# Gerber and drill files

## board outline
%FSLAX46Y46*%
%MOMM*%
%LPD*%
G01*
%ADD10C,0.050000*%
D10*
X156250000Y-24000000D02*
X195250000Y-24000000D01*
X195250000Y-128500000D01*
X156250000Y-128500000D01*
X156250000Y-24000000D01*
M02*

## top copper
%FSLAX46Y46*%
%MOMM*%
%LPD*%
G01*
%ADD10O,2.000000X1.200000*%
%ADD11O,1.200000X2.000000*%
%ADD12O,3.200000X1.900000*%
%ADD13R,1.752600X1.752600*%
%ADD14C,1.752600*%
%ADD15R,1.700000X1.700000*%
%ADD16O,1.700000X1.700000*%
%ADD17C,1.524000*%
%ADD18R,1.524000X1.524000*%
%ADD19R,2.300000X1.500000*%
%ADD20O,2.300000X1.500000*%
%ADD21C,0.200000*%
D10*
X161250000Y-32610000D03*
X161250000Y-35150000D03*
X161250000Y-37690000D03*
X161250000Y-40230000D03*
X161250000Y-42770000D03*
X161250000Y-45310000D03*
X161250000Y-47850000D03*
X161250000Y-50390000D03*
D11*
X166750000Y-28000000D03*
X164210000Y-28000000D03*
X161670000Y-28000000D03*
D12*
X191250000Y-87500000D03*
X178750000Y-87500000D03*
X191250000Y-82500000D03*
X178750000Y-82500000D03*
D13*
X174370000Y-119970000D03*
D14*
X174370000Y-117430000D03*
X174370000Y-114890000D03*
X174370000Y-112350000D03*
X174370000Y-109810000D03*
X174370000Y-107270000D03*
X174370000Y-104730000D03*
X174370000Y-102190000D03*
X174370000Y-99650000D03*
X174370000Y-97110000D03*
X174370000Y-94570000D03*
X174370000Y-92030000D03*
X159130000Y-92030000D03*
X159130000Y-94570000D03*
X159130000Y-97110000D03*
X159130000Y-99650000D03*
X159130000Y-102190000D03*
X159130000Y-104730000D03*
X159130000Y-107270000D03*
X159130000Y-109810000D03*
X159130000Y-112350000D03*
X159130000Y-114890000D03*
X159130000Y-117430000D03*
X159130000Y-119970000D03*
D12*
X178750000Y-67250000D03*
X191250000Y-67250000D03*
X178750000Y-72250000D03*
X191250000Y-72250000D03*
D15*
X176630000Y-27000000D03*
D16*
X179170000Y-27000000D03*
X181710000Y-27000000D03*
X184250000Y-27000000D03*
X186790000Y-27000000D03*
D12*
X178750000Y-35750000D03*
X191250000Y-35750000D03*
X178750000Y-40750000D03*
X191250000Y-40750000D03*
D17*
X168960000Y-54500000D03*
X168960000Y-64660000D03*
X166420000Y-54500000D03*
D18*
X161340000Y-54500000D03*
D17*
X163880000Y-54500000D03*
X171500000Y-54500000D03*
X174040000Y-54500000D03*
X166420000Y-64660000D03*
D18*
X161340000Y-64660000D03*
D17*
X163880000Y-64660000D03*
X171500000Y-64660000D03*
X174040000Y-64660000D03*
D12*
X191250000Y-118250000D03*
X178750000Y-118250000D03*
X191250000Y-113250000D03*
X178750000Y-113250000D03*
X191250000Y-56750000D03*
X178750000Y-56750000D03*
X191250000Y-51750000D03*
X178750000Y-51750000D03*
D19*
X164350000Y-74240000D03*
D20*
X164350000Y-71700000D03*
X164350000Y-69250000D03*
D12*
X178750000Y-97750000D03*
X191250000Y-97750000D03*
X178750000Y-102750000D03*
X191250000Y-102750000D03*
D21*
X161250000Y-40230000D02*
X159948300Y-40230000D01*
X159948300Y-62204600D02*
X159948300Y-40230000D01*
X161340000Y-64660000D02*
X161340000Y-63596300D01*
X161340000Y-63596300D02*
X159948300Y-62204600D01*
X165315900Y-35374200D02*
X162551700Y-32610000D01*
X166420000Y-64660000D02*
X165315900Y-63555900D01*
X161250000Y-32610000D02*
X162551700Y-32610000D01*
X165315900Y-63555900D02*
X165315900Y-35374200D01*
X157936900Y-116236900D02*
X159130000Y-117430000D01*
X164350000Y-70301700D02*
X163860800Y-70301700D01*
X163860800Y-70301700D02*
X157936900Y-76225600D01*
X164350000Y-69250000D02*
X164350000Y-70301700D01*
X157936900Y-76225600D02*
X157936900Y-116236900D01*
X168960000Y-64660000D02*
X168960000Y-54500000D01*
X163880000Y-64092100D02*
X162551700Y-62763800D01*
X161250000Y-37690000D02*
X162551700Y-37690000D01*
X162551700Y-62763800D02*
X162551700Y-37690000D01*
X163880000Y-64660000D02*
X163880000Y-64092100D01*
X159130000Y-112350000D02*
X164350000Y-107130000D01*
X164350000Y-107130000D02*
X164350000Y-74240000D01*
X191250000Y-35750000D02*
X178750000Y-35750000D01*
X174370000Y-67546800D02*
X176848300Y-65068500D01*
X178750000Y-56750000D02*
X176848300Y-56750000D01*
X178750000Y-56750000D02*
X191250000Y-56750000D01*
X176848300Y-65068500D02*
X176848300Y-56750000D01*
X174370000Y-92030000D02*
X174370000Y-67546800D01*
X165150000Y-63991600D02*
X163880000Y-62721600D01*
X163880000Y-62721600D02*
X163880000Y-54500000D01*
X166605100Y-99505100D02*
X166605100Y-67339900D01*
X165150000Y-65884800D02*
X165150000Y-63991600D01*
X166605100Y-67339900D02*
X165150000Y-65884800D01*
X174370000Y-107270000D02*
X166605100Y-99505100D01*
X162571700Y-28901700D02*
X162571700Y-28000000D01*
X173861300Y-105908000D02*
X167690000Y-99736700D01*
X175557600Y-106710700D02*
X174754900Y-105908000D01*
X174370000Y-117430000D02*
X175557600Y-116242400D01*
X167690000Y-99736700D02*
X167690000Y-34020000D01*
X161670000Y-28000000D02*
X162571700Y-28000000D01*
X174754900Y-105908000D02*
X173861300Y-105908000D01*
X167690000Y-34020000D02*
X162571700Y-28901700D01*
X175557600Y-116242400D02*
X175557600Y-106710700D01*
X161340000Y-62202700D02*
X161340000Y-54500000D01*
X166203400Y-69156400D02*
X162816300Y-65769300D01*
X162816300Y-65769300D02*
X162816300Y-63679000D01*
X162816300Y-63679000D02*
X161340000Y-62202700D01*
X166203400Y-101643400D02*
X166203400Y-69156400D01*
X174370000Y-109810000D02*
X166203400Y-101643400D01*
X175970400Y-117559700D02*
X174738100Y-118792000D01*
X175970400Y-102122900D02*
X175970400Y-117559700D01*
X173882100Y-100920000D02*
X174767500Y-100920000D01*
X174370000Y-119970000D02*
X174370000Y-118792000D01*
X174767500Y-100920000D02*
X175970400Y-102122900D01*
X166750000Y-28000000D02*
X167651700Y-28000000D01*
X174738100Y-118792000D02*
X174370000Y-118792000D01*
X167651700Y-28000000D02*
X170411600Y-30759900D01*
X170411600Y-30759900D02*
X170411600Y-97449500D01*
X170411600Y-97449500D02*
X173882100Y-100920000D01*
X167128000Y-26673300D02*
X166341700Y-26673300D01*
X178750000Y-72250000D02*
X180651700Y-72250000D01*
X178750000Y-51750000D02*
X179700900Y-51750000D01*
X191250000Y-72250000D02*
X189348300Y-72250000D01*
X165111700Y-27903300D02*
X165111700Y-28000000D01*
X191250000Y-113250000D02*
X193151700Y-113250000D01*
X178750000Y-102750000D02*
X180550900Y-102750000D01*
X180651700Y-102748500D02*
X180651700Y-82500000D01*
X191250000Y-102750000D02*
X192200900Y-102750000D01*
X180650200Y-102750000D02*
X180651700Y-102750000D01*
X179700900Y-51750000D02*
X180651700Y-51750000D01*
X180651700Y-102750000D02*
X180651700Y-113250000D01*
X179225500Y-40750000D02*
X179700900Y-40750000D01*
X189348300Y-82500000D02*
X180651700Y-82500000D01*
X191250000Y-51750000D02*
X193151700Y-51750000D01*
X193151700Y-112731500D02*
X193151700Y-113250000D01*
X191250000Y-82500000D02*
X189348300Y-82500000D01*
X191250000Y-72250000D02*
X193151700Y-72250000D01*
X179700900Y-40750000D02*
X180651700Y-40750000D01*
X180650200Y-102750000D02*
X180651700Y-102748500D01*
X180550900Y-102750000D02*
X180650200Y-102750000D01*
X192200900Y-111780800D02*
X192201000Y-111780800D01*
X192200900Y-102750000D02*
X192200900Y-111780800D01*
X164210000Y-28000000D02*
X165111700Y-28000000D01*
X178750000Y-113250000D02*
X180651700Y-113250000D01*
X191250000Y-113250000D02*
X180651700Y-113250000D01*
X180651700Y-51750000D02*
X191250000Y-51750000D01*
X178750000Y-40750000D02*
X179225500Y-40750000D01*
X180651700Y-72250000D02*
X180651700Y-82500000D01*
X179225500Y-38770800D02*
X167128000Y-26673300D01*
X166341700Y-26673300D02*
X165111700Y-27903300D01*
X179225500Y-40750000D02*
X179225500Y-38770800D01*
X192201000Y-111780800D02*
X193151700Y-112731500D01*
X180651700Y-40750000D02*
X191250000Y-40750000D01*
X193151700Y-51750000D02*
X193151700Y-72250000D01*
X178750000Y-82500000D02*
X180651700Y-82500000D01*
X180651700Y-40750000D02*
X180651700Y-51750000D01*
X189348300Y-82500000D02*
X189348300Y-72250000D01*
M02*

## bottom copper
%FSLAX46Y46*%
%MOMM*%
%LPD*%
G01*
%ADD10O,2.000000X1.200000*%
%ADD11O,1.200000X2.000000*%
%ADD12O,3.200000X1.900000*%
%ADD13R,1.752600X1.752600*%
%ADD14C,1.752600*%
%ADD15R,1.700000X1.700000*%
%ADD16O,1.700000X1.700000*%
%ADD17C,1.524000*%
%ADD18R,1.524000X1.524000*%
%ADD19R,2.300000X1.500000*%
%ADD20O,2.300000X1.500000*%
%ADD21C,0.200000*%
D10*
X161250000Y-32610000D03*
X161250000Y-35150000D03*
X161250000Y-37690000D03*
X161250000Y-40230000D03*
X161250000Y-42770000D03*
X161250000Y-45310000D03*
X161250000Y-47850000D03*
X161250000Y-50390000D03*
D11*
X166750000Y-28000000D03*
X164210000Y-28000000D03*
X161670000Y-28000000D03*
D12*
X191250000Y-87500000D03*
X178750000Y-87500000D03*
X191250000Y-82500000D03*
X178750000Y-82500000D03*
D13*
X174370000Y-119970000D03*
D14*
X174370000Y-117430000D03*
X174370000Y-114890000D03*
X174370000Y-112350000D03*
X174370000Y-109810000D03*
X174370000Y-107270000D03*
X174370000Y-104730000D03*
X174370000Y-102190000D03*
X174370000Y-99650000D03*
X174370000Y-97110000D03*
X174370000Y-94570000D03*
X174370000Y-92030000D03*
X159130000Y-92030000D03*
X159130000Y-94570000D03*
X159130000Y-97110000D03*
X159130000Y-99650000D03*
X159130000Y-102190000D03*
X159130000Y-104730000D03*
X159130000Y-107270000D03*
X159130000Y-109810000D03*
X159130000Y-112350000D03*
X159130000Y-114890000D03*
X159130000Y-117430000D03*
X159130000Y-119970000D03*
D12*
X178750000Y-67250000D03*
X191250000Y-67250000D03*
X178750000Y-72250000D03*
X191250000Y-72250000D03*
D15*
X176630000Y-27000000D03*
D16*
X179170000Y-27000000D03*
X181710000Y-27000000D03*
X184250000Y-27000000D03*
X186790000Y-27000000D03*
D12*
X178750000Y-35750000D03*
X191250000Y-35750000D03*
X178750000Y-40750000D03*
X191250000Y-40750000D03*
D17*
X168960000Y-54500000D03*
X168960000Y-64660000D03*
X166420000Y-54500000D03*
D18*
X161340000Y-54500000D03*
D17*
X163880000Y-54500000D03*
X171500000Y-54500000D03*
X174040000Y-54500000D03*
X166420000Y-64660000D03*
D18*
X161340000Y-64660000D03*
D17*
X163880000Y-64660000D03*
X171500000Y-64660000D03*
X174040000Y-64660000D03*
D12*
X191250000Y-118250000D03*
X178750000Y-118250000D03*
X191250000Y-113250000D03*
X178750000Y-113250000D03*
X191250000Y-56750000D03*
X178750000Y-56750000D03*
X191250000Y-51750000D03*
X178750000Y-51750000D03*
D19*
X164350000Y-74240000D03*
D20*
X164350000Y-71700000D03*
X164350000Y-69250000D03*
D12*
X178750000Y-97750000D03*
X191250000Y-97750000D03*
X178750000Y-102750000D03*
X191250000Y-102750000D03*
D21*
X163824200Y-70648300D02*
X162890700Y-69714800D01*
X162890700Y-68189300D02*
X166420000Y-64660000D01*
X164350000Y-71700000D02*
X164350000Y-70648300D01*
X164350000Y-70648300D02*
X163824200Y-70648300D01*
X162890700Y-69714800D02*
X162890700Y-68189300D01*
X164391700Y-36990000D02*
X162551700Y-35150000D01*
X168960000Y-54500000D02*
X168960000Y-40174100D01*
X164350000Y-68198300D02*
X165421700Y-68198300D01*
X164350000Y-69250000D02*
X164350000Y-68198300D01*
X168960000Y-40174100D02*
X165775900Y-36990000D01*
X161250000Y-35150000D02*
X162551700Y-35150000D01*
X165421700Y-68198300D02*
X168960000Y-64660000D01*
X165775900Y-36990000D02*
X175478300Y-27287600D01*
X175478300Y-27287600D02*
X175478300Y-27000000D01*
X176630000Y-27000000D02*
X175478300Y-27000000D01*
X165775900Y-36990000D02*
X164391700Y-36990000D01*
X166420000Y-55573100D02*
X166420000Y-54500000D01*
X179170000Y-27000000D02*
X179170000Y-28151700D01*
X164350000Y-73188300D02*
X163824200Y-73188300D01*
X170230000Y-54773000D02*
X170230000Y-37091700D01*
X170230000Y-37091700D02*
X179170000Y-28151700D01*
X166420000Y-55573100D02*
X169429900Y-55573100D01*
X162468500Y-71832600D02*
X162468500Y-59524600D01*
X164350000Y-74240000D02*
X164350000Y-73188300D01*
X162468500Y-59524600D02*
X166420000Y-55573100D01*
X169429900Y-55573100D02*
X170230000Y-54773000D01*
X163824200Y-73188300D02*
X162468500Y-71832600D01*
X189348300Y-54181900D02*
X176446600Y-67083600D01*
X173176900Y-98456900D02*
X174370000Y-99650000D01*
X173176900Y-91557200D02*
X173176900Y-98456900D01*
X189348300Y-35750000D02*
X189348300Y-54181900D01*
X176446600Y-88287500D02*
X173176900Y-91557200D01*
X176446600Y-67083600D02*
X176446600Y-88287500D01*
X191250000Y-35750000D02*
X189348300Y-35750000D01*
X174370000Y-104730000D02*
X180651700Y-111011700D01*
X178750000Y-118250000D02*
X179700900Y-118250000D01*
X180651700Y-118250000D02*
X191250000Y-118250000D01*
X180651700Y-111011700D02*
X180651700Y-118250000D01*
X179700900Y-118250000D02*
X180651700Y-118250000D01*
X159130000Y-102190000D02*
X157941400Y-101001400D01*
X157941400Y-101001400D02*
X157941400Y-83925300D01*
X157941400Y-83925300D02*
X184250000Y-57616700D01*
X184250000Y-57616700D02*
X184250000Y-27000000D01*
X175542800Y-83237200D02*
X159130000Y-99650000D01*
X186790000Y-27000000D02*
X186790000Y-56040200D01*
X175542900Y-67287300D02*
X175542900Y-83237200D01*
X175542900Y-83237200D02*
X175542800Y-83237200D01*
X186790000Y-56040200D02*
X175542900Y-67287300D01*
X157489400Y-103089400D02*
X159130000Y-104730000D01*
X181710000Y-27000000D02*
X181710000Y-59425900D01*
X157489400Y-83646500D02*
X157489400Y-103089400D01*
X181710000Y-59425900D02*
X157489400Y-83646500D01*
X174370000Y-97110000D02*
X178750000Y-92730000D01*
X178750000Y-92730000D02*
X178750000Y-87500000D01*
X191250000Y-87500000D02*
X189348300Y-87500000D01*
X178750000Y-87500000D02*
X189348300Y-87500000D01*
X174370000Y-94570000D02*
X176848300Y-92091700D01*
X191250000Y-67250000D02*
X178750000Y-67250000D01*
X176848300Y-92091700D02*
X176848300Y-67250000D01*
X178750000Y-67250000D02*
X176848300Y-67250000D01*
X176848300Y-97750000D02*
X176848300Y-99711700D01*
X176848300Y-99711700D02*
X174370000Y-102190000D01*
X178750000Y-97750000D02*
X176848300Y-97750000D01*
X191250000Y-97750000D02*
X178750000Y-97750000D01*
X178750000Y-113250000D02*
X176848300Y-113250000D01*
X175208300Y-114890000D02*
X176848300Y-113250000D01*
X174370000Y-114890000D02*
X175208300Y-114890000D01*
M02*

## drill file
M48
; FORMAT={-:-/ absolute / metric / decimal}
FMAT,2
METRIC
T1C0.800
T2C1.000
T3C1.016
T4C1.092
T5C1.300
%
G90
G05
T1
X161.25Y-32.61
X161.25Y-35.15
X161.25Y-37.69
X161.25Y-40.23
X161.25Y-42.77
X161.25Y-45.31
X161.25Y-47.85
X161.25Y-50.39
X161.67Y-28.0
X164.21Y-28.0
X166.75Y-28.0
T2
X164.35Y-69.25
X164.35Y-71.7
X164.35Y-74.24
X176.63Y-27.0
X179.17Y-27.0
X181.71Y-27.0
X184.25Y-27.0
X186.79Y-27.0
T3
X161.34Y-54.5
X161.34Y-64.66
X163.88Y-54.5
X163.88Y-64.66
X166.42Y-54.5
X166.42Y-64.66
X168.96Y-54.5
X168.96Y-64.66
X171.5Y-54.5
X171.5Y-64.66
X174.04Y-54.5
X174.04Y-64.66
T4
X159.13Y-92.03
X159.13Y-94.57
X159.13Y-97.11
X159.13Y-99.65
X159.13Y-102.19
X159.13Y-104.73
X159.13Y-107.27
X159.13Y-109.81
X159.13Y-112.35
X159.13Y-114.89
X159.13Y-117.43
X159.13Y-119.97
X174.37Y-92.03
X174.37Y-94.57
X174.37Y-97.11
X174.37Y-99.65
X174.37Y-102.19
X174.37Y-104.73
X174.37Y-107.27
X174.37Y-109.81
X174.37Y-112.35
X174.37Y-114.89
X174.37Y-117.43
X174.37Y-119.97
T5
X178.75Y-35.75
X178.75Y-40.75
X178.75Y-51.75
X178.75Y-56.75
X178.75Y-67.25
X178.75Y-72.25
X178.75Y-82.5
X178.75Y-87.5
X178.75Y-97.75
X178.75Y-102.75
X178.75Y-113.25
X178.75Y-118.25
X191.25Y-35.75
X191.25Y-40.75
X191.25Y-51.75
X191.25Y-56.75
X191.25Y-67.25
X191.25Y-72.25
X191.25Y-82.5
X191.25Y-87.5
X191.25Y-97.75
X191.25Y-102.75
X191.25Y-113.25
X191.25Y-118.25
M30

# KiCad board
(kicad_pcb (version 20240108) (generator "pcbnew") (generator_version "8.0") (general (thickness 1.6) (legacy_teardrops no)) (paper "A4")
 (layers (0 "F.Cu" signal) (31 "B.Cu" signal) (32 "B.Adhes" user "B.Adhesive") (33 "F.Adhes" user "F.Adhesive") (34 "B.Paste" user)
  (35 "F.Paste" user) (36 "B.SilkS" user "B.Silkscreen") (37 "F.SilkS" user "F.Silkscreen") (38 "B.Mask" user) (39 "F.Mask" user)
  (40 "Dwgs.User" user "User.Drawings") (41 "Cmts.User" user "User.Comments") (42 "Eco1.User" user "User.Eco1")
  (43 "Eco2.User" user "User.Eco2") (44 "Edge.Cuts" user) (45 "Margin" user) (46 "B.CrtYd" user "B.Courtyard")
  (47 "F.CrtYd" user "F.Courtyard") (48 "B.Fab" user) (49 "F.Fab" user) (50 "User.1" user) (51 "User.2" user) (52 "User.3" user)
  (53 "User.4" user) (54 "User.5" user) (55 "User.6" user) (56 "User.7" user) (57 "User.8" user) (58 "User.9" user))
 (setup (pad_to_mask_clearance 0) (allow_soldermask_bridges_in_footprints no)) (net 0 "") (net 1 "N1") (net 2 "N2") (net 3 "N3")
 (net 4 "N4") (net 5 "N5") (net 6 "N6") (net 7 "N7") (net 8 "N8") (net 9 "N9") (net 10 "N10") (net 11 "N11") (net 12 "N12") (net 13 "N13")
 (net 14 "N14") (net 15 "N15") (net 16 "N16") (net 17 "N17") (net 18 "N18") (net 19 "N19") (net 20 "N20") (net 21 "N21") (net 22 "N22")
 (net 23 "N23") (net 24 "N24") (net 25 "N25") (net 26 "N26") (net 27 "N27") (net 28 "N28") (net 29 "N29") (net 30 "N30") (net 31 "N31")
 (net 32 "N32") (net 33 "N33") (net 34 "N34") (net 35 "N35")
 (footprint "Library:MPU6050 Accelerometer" (layer "F.Cu") (at 167.75 43.75)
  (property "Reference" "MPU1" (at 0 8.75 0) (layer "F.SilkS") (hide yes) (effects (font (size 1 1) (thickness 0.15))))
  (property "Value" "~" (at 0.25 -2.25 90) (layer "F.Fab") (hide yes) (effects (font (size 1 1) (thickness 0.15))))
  (pad "1" thru_hole oval (at -6.5 -11.14 270) (size 1.2 2) (drill 0.8) (layers "*.Cu" "*.Mask") (remove_unused_layers no) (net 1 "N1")
   (thermal_bridge_angle 45))
  (pad "2" thru_hole oval (at -6.5 -8.6 270) (size 1.2 2) (drill 0.8) (layers "*.Cu" "*.Mask") (remove_unused_layers no) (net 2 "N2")
   (thermal_bridge_angle 45))
  (pad "3" thru_hole oval (at -6.5 -6.06 270) (size 1.2 2) (drill 0.8) (layers "*.Cu" "*.Mask") (remove_unused_layers no) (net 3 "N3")
   (thermal_bridge_angle 45))
  (pad "4" thru_hole oval (at -6.5 -3.52 270) (size 1.2 2) (drill 0.8) (layers "*.Cu" "*.Mask") (remove_unused_layers no) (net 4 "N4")
   (thermal_bridge_angle 45))
  (pad "5" thru_hole oval (at -6.5 -0.98 270) (size 1.2 2) (drill 0.8) (layers "*.Cu" "*.Mask") (remove_unused_layers no) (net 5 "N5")
   (thermal_bridge_angle 45))
  (pad "6" thru_hole oval (at -6.5 1.56 270) (size 1.2 2) (drill 0.8) (layers "*.Cu" "*.Mask") (remove_unused_layers no) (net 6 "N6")
   (thermal_bridge_angle 45))
  (pad "7" thru_hole oval (at -6.5 4.1 270) (size 1.2 2) (drill 0.8) (layers "*.Cu" "*.Mask") (remove_unused_layers no) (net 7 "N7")
   (thermal_bridge_angle 45))
  (pad "8" thru_hole oval (at -6.5 6.64 270) (size 1.2 2) (drill 0.8) (layers "*.Cu" "*.Mask") (remove_unused_layers no) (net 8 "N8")
   (thermal_bridge_angle 45)))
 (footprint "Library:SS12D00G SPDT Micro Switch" (layer "F.Cu") (at 164.21 28 180)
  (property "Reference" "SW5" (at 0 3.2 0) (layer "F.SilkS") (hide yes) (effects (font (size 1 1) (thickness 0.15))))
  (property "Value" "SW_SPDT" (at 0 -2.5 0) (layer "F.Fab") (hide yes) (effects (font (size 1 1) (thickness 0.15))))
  (pad "1" thru_hole oval (at -2.54 0 180) (size 1.2 2) (drill 0.8) (layers "*.Cu" "*.Mask") (remove_unused_layers no) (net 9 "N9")
   (thermal_bridge_angle 45))
  (pad "2" thru_hole oval (at 0 0 180) (size 1.2 2) (drill 0.8) (layers "*.Cu" "*.Mask") (remove_unused_layers no) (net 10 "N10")
   (thermal_bridge_angle 45))
  (pad "3" thru_hole oval (at 2.54 0 180) (size 1.2 2) (drill 0.8) (layers "*.Cu" "*.Mask") (remove_unused_layers no) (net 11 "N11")
   (thermal_bridge_angle 45)))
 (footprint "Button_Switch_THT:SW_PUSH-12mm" (layer "F.Cu") (at 191.25 87.5 180)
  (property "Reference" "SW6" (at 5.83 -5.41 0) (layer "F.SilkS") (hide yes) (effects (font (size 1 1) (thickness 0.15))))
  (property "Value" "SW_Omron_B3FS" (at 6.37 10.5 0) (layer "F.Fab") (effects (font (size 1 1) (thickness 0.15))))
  (pad "1" thru_hole oval (at 0 0 180) (size 3.2 1.9) (drill 1.3) (layers "*.Cu" "*.Mask") (remove_unused_layers no) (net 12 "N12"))
  (pad "1" thru_hole oval (at 12.5 0 180) (size 3.2 1.9) (drill 1.3) (layers "*.Cu" "*.Mask") (remove_unused_layers no) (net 12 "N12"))
  (pad "2" thru_hole oval (at 0 5 180) (size 3.2 1.9) (drill 1.3) (layers "*.Cu" "*.Mask") (remove_unused_layers no) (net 10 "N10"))
  (pad "2" thru_hole oval (at 12.5 5 180) (size 3.2 1.9) (drill 1.3) (layers "*.Cu" "*.Mask") (remove_unused_layers no) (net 10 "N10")))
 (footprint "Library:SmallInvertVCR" (layer "F.Cu") (at 167 83.5)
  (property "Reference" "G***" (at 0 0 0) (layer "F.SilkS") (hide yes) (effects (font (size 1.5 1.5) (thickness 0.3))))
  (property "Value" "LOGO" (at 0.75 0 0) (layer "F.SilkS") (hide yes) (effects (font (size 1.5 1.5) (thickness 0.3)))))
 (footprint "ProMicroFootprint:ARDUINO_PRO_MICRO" (layer "F.Cu") (at 166.75 106 90)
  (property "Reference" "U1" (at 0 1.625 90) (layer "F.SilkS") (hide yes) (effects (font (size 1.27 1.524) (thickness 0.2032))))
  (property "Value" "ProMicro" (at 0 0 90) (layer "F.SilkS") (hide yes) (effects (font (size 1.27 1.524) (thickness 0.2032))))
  (pad "1" thru_hole rect (at -13.97 7.62 90) (size 1.7526 1.7526) (drill 1.0922) (layers "*.Cu" "*.SilkS" "*.Mask")
   (remove_unused_layers no) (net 9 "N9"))
  (pad "2" thru_hole circle (at -11.43 7.62 90) (size 1.7526 1.7526) (drill 1.0922) (layers "*.Cu" "*.SilkS" "*.Mask")
   (remove_unused_layers no) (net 11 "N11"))
  (pad "3" thru_hole circle (at -8.89 7.62 90) (size 1.7526 1.7526) (drill 1.0922) (layers "*.Cu" "*.SilkS" "*.Mask")
   (remove_unused_layers no) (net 10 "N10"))
  (pad "4" thru_hole circle (at -6.35 7.62 90) (size 1.7526 1.7526) (drill 1.0922) (layers "*.Cu" "*.SilkS" "*.Mask")
   (remove_unused_layers no) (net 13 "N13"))
  (pad "5" thru_hole circle (at -3.81 7.62 90) (size 1.7526 1.7526) (drill 1.0922) (layers "*.Cu" "*.SilkS" "*.Mask")
   (remove_unused_layers no) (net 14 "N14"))
  (pad "6" thru_hole circle (at -1.27 7.62 90) (size 1.7526 1.7526) (drill 1.0922) (layers "*.Cu" "*.SilkS" "*.Mask")
   (remove_unused_layers no) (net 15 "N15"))
  (pad "7" thru_hole circle (at 1.27 7.62 90) (size 1.7526 1.7526) (drill 1.0922) (layers "*.Cu" "*.SilkS" "*.Mask")
   (remove_unused_layers no) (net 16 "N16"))
  (pad "8" thru_hole circle (at 3.81 7.62 90) (size 1.7526 1.7526) (drill 1.0922) (layers "*.Cu" "*.SilkS" "*.Mask")
   (remove_unused_layers no) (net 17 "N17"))
  (pad "9" thru_hole circle (at 6.35 7.62 90) (size 1.7526 1.7526) (drill 1.0922) (layers "*.Cu" "*.SilkS" "*.Mask")
   (remove_unused_layers no) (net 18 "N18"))
  (pad "10" thru_hole circle (at 8.89 7.62 90) (size 1.7526 1.7526) (drill 1.0922) (layers "*.Cu" "*.SilkS" "*.Mask")
   (remove_unused_layers no) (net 12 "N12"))
  (pad "11" thru_hole circle (at 11.43 7.62 90) (size 1.7526 1.7526) (drill 1.0922) (layers "*.Cu" "*.SilkS" "*.Mask")
   (remove_unused_layers no) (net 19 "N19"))
  (pad "12" thru_hole circle (at 13.97 7.62 90) (size 1.7526 1.7526) (drill 1.0922) (layers "*.Cu" "*.SilkS" "*.Mask")
   (remove_unused_layers no) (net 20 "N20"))
  (pad "13" thru_hole circle (at 13.97 -7.62 90) (size 1.7526 1.7526) (drill 1.0922) (layers "*.Cu" "*.SilkS" "*.Mask")
   (remove_unused_layers no) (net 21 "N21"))
  (pad "14" thru_hole circle (at 11.43 -7.62 90) (size 1.7526 1.7526) (drill 1.0922) (layers "*.Cu" "*.SilkS" "*.Mask")
   (remove_unused_layers no) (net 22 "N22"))
  (pad "15" thru_hole circle (at 8.89 -7.62 90) (size 1.7526 1.7526) (drill 1.0922) (layers "*.Cu" "*.SilkS" "*.Mask")
   (remove_unused_layers no) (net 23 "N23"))
  (pad "16" thru_hole circle (at 6.35 -7.62 90) (size 1.7526 1.7526) (drill 1.0922) (layers "*.Cu" "*.SilkS" "*.Mask")
   (remove_unused_layers no) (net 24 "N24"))
  (pad "17" thru_hole circle (at 3.81 -7.62 90) (size 1.7526 1.7526) (drill 1.0922) (layers "*.Cu" "*.SilkS" "*.Mask")
   (remove_unused_layers no) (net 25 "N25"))
  (pad "18" thru_hole circle (at 1.27 -7.62 90) (size 1.7526 1.7526) (drill 1.0922) (layers "*.Cu" "*.SilkS" "*.Mask")
   (remove_unused_layers no) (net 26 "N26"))
  (pad "19" thru_hole circle (at -1.27 -7.62 90) (size 1.7526 1.7526) (drill 1.0922) (layers "*.Cu" "*.SilkS" "*.Mask")
   (remove_unused_layers no) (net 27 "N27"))
  (pad "20" thru_hole circle (at -3.81 -7.62 90) (size 1.7526 1.7526) (drill 1.0922) (layers "*.Cu" "*.SilkS" "*.Mask")
   (remove_unused_layers no) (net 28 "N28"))
  (pad "21" thru_hole circle (at -6.35 -7.62 90) (size 1.7526 1.7526) (drill 1.0922) (layers "*.Cu" "*.SilkS" "*.Mask")
   (remove_unused_layers no) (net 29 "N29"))
  (pad "22" thru_hole circle (at -8.89 -7.62 90) (size 1.7526 1.7526) (drill 1.0922) (layers "*.Cu" "*.SilkS" "*.Mask")
   (remove_unused_layers no) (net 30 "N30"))
  (pad "23" thru_hole circle (at -11.43 -7.62 90) (size 1.7526 1.7526) (drill 1.0922) (layers "*.Cu" "*.SilkS" "*.Mask")
   (remove_unused_layers no) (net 2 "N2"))
  (pad "24" thru_hole circle (at -13.97 -7.62 90) (size 1.7526 1.7526) (drill 1.0922) (layers "*.Cu" "*.SilkS" "*.Mask")
   (remove_unused_layers no) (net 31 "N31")))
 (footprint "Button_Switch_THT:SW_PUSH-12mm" (layer "F.Cu") (at 178.75 67.25)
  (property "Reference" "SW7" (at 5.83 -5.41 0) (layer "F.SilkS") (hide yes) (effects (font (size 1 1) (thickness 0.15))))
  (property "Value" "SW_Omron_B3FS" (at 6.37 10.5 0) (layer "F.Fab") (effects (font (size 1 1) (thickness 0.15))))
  (pad "1" thru_hole oval (at 0 0) (size 3.2 1.9) (drill 1.3) (layers "*.Cu" "*.Mask") (remove_unused_layers no) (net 19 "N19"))
  (pad "1" thru_hole oval (at 12.5 0) (size 3.2 1.9) (drill 1.3) (layers "*.Cu" "*.Mask") (remove_unused_layers no) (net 19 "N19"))
  (pad "2" thru_hole oval (at 0 5) (size 3.2 1.9) (drill 1.3) (layers "*.Cu" "*.Mask") (remove_unused_layers no) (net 10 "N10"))
  (pad "2" thru_hole oval (at 12.5 5) (size 3.2 1.9) (drill 1.3) (layers "*.Cu" "*.Mask") (remove_unused_layers no) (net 10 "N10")))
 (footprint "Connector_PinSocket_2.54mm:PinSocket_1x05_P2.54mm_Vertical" (layer "F.Cu") (at 176.63 27 90)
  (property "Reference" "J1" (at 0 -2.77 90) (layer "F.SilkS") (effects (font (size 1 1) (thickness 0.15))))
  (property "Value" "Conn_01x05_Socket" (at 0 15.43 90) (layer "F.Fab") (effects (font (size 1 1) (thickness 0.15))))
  (pad "1" thru_hole rect (at 0 0 90) (size 1.7 1.7) (drill 1) (layers "*.Cu" "*.Mask") (remove_unused_layers no) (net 2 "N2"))
  (pad "2" thru_hole oval (at 0 2.54 90) (size 1.7 1.7) (drill 1) (layers "*.Cu" "*.Mask") (remove_unused_layers no) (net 29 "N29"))
  (pad "3" thru_hole oval (at 0 5.08 90) (size 1.7 1.7) (drill 1) (layers "*.Cu" "*.Mask") (remove_unused_layers no) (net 26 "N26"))
  (pad "4" thru_hole oval (at 0 7.62 90) (size 1.7 1.7) (drill 1) (layers "*.Cu" "*.Mask") (remove_unused_layers no) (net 25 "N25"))
  (pad "5" thru_hole oval (at 0 10.16 90) (size 1.7 1.7) (drill 1) (layers "*.Cu" "*.Mask") (remove_unused_layers no) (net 24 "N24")))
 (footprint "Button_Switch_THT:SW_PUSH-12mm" (layer "F.Cu") (at 178.75 35.75)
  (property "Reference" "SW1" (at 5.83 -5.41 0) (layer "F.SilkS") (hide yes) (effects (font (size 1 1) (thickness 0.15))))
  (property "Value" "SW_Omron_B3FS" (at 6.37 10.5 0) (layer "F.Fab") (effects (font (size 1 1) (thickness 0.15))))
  (pad "1" thru_hole oval (at 0 0) (size 3.2 1.9) (drill 1.3) (layers "*.Cu" "*.Mask") (remove_unused_layers no) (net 18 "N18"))
  (pad "1" thru_hole oval (at 12.5 0) (size 3.2 1.9) (drill 1.3) (layers "*.Cu" "*.Mask") (remove_unused_layers no) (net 18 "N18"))
  (pad "2" thru_hole oval (at 0 5) (size 3.2 1.9) (drill 1.3) (layers "*.Cu" "*.Mask") (remove_unused_layers no) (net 10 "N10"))
  (pad "2" thru_hole oval (at 12.5 5) (size 3.2 1.9) (drill 1.3) (layers "*.Cu" "*.Mask") (remove_unused_layers no) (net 10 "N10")))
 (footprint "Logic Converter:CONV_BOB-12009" (layer "F.Cu") (at 167.69 59.58 90)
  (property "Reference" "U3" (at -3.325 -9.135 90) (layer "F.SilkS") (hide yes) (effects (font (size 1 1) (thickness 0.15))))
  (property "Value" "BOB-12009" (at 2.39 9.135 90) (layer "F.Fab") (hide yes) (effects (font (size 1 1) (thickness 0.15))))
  (pad "GND_1" thru_hole circle (at 5.08 1.27 90) (size 1.524 1.524) (drill 1.016) (layers "*.Cu" "*.Mask") (remove_unused_layers no)
   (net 2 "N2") (solder_mask_margin 0.102))
  (pad "GND_2" thru_hole circle (at -5.08 1.27 90) (size 1.524 1.524) (drill 1.016) (layers "*.Cu" "*.Mask") (remove_unused_layers no)
   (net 2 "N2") (solder_mask_margin 0.102))
  (pad "HV" thru_hole circle (at 5.08 -1.27 90) (size 1.524 1.524) (drill 1.016) (layers "*.Cu" "*.Mask") (remove_unused_layers no)
   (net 29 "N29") (solder_mask_margin 0.102))
  (pad "HV1" thru_hole rect (at 5.08 -6.35 90) (size 1.524 1.524) (drill 1.016) (layers "*.Cu" "*.Mask") (remove_unused_layers no)
   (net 14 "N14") (solder_mask_margin 0.102))
  (pad "HV2" thru_hole circle (at 5.08 -3.81 90) (size 1.524 1.524) (drill 1.016) (layers "*.Cu" "*.Mask") (remove_unused_layers no)
   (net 15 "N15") (solder_mask_margin 0.102))
  (pad "HV3" thru_hole circle (at 5.08 3.81 90) (size 1.524 1.524) (drill 1.016) (layers "*.Cu" "*.Mask") (remove_unused_layers no)
   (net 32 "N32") (solder_mask_margin 0.102))
  (pad "HV4" thru_hole circle (at 5.08 6.35 90) (size 1.524 1.524) (drill 1.016) (layers "*.Cu" "*.Mask") (remove_unused_layers no)
   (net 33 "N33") (solder_mask_margin 0.102))
  (pad "LV" thru_hole circle (at -5.08 -1.27 90) (size 1.524 1.524) (drill 1.016) (layers "*.Cu" "*.Mask") (remove_unused_layers no)
   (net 1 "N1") (solder_mask_margin 0.102))
  (pad "LV1" thru_hole rect (at -5.08 -6.35 90) (size 1.524 1.524) (drill 1.016) (layers "*.Cu" "*.Mask") (remove_unused_layers no)
   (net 4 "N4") (solder_mask_margin 0.102))
  (pad "LV2" thru_hole circle (at -5.08 -3.81 90) (size 1.524 1.524) (drill 1.016) (layers "*.Cu" "*.Mask") (remove_unused_layers no)
   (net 3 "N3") (solder_mask_margin 0.102))
  (pad "LV3" thru_hole circle (at -5.08 3.81 90) (size 1.524 1.524) (drill 1.016) (layers "*.Cu" "*.Mask") (remove_unused_layers no)
   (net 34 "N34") (solder_mask_margin 0.102))
  (pad "LV4" thru_hole circle (at -5.08 6.35 90) (size 1.524 1.524) (drill 1.016) (layers "*.Cu" "*.Mask") (remove_unused_layers no)
   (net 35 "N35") (solder_mask_margin 0.102)))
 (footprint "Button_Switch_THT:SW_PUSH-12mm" (layer "F.Cu") (at 191.25 118.25 180)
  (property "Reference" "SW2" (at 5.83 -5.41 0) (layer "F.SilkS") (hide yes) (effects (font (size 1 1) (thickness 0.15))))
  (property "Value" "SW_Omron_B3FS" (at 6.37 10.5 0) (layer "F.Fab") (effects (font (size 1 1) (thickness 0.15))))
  (pad "1" thru_hole oval (at 0 0 180) (size 3.2 1.9) (drill 1.3) (layers "*.Cu" "*.Mask") (remove_unused_layers no) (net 16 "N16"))
  (pad "1" thru_hole oval (at 12.5 0 180) (size 3.2 1.9) (drill 1.3) (layers "*.Cu" "*.Mask") (remove_unused_layers no) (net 16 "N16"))
  (pad "2" thru_hole oval (at 0 5 180) (size 3.2 1.9) (drill 1.3) (layers "*.Cu" "*.Mask") (remove_unused_layers no) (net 10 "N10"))
  (pad "2" thru_hole oval (at 12.5 5 180) (size 3.2 1.9) (drill 1.3) (layers "*.Cu" "*.Mask") (remove_unused_layers no) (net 10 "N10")))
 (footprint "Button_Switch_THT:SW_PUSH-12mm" (layer "F.Cu") (at 191.25 56.75 180)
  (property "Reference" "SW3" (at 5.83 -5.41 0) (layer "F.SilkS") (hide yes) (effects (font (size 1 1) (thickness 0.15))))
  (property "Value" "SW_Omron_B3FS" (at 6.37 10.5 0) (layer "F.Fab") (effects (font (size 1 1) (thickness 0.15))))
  (pad "1" thru_hole oval (at 0 0 180) (size 3.2 1.9) (drill 1.3) (layers "*.Cu" "*.Mask") (remove_unused_layers no) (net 20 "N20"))
  (pad "1" thru_hole oval (at 12.5 0 180) (size 3.2 1.9) (drill 1.3) (layers "*.Cu" "*.Mask") (remove_unused_layers no) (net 20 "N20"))
  (pad "2" thru_hole oval (at 0 5 180) (size 3.2 1.9) (drill 1.3) (layers "*.Cu" "*.Mask") (remove_unused_layers no) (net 10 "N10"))
  (pad "2" thru_hole oval (at 12.5 5 180) (size 3.2 1.9) (drill 1.3) (layers "*.Cu" "*.Mask") (remove_unused_layers no) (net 10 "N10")))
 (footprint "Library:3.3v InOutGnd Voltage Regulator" (layer "F.Cu") (at 162.85 71.75 -90)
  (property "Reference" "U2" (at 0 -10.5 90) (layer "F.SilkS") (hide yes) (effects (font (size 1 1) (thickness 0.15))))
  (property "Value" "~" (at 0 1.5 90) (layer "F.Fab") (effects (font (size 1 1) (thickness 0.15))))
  (pad "1" thru_hole rect (at 2.49 -1.5 270) (size 1.5 2.3) (drill 1) (layers "*.Cu" "*.Mask") (remove_unused_layers no) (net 29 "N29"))
  (pad "2" thru_hole oval (at -0.05 -1.5 270) (size 1.5 2.3) (drill 1) (layers "*.Cu" "*.Mask") (remove_unused_layers no) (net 1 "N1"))
  (pad "3" thru_hole oval (at -2.5 -1.5 270) (size 1.5 2.3) (drill 1) (layers "*.Cu" "*.Mask") (remove_unused_layers no) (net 2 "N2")))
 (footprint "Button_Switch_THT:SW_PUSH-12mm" (layer "F.Cu") (at 178.75 97.75)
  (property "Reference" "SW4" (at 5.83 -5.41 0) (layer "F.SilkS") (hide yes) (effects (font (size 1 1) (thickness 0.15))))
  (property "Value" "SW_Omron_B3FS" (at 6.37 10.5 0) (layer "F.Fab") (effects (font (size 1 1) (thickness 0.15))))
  (pad "1" thru_hole oval (at 0 0) (size 3.2 1.9) (drill 1.3) (layers "*.Cu" "*.Mask") (remove_unused_layers no) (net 17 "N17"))
  (pad "1" thru_hole oval (at 12.5 0) (size 3.2 1.9) (drill 1.3) (layers "*.Cu" "*.Mask") (remove_unused_layers no) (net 17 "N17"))
  (pad "2" thru_hole oval (at 0 5) (size 3.2 1.9) (drill 1.3) (layers "*.Cu" "*.Mask") (remove_unused_layers no) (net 10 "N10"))
  (pad "2" thru_hole oval (at 12.5 5) (size 3.2 1.9) (drill 1.3) (layers "*.Cu" "*.Mask") (remove_unused_layers no) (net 10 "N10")))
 (gr_rect (start 156.25 24) (end 195.25 128.5) (stroke (width 0.05) (type default)) (fill none) (layer "Edge.Cuts"))
 (segment (start 161.25 40.23) (end 159.9483 40.23) (width 0.2) (layer "F.Cu") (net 4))
 (segment (start 159.9483 62.2046) (end 159.9483 40.23) (width 0.2) (layer "F.Cu") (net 4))
 (segment (start 161.34 64.66) (end 161.34 63.5963) (width 0.2) (layer "F.Cu") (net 4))
 (segment (start 161.34 63.5963) (end 159.9483 62.2046) (width 0.2) (layer "F.Cu") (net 4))
 (segment (start 165.3159 35.3742) (end 162.5517 32.61) (width 0.2) (layer "F.Cu") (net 1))
 (segment (start 166.42 64.66) (end 165.3159 63.5559) (width 0.2) (layer "F.Cu") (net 1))
 (segment (start 161.25 32.61) (end 162.5517 32.61) (width 0.2) (layer "F.Cu") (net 1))
 (segment (start 165.3159 63.5559) (end 165.3159 35.3742) (width 0.2) (layer "F.Cu") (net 1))
 (segment (start 163.8242 70.6483) (end 162.8907 69.7148) (width 0.2) (layer "B.Cu") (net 1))
 (segment (start 162.8907 68.1893) (end 166.42 64.66) (width 0.2) (layer "B.Cu") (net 1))
 (segment (start 164.35 71.7) (end 164.35 70.6483) (width 0.2) (layer "B.Cu") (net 1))
 (segment (start 164.35 70.6483) (end 163.8242 70.6483) (width 0.2) (layer "B.Cu") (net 1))
 (segment (start 162.8907 69.7148) (end 162.8907 68.1893) (width 0.2) (layer "B.Cu") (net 1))
 (segment (start 157.9369 116.2369) (end 159.13 117.43) (width 0.2) (layer "F.Cu") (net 2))
 (segment (start 164.35 70.3017) (end 163.8608 70.3017) (width 0.2) (layer "F.Cu") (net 2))
 (segment (start 163.8608 70.3017) (end 157.9369 76.2256) (width 0.2) (layer "F.Cu") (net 2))
 (segment (start 164.35 69.25) (end 164.35 70.3017) (width 0.2) (layer "F.Cu") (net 2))
 (segment (start 157.9369 76.2256) (end 157.9369 116.2369) (width 0.2) (layer "F.Cu") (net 2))
 (segment (start 168.96 64.66) (end 168.96 54.5) (width 0.2) (layer "F.Cu") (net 2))
 (segment (start 164.3917 36.99) (end 162.5517 35.15) (width 0.2) (layer "B.Cu") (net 2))
 (segment (start 168.96 54.5) (end 168.96 40.1741) (width 0.2) (layer "B.Cu") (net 2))
 (segment (start 164.35 68.1983) (end 165.4217 68.1983) (width 0.2) (layer "B.Cu") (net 2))
 (segment (start 164.35 69.25) (end 164.35 68.1983) (width 0.2) (layer "B.Cu") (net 2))
 (segment (start 168.96 40.1741) (end 165.7759 36.99) (width 0.2) (layer "B.Cu") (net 2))
 (segment (start 161.25 35.15) (end 162.5517 35.15) (width 0.2) (layer "B.Cu") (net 2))
 (segment (start 165.4217 68.1983) (end 168.96 64.66) (width 0.2) (layer "B.Cu") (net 2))
 (segment (start 165.7759 36.99) (end 175.4783 27.2876) (width 0.2) (layer "B.Cu") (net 2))
 (segment (start 175.4783 27.2876) (end 175.4783 27) (width 0.2) (layer "B.Cu") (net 2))
 (segment (start 176.63 27) (end 175.4783 27) (width 0.2) (layer "B.Cu") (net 2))
 (segment (start 165.7759 36.99) (end 164.3917 36.99) (width 0.2) (layer "B.Cu") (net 2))
 (segment (start 163.88 64.0921) (end 162.5517 62.7638) (width 0.2) (layer "F.Cu") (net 3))
 (segment (start 161.25 37.69) (end 162.5517 37.69) (width 0.2) (layer "F.Cu") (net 3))
 (segment (start 162.5517 62.7638) (end 162.5517 37.69) (width 0.2) (layer "F.Cu") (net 3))
 (segment (start 163.88 64.66) (end 163.88 64.0921) (width 0.2) (layer "F.Cu") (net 3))
 (segment (start 159.13 112.35) (end 164.35 107.13) (width 0.2) (layer "F.Cu") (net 29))
 (segment (start 164.35 107.13) (end 164.35 74.24) (width 0.2) (layer "F.Cu") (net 29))
 (segment (start 166.42 55.5731) (end 166.42 54.5) (width 0.2) (layer "B.Cu") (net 29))
 (segment (start 179.17 27) (end 179.17 28.1517) (width 0.2) (layer "B.Cu") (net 29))
 (segment (start 164.35 73.1883) (end 163.8242 73.1883) (width 0.2) (layer "B.Cu") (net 29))
 (segment (start 170.23 54.773) (end 170.23 37.0917) (width 0.2) (layer "B.Cu") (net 29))
 (segment (start 170.23 37.0917) (end 179.17 28.1517) (width 0.2) (layer "B.Cu") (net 29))
 (segment (start 166.42 55.5731) (end 169.4299 55.5731) (width 0.2) (layer "B.Cu") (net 29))
 (segment (start 162.4685 71.8326) (end 162.4685 59.5246) (width 0.2) (layer "B.Cu") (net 29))
 (segment (start 164.35 74.24) (end 164.35 73.1883) (width 0.2) (layer "B.Cu") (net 29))
 (segment (start 162.4685 59.5246) (end 166.42 55.5731) (width 0.2) (layer "B.Cu") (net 29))
 (segment (start 169.4299 55.5731) (end 170.23 54.773) (width 0.2) (layer "B.Cu") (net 29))
 (segment (start 163.8242 73.1883) (end 162.4685 71.8326) (width 0.2) (layer "B.Cu") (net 29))
 (segment (start 191.25 35.75) (end 178.75 35.75) (width 0.2) (layer "F.Cu") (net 18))
 (segment (start 189.3483 54.1819) (end 176.4466 67.0836) (width 0.2) (layer "B.Cu") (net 18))
 (segment (start 173.1769 98.4569) (end 174.37 99.65) (width 0.2) (layer "B.Cu") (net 18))
 (segment (start 173.1769 91.5572) (end 173.1769 98.4569) (width 0.2) (layer "B.Cu") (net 18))
 (segment (start 189.3483 35.75) (end 189.3483 54.1819) (width 0.2) (layer "B.Cu") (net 18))
 (segment (start 176.4466 88.2875) (end 173.1769 91.5572) (width 0.2) (layer "B.Cu") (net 18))
 (segment (start 176.4466 67.0836) (end 176.4466 88.2875) (width 0.2) (layer "B.Cu") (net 18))
 (segment (start 191.25 35.75) (end 189.3483 35.75) (width 0.2) (layer "B.Cu") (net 18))
 (segment (start 174.37 104.73) (end 180.6517 111.0117) (width 0.2) (layer "B.Cu") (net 16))
 (segment (start 178.75 118.25) (end 179.7009 118.25) (width 0.2) (layer "B.Cu") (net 16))
 (segment (start 180.6517 118.25) (end 191.25 118.25) (width 0.2) (layer "B.Cu") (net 16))
 (segment (start 180.6517 111.0117) (end 180.6517 118.25) (width 0.2) (layer "B.Cu") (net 16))
 (segment (start 179.7009 118.25) (end 180.6517 118.25) (width 0.2) (layer "B.Cu") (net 16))
 (segment (start 174.37 67.5468) (end 176.8483 65.0685) (width 0.2) (layer "F.Cu") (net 20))
 (segment (start 178.75 56.75) (end 176.8483 56.75) (width 0.2) (layer "F.Cu") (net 20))
 (segment (start 178.75 56.75) (end 191.25 56.75) (width 0.2) (layer "F.Cu") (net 20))
 (segment (start 176.8483 65.0685) (end 176.8483 56.75) (width 0.2) (layer "F.Cu") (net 20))
 (segment (start 174.37 92.03) (end 174.37 67.5468) (width 0.2) (layer "F.Cu") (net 20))
 (segment (start 159.13 102.19) (end 157.9414 101.0014) (width 0.2) (layer "B.Cu") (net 25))
 (segment (start 157.9414 101.0014) (end 157.9414 83.9253) (width 0.2) (layer "B.Cu") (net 25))
 (segment (start 157.9414 83.9253) (end 184.25 57.6167) (width 0.2) (layer "B.Cu") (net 25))
 (segment (start 184.25 57.6167) (end 184.25 27) (width 0.2) (layer "B.Cu") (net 25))
 (segment (start 175.5428 83.2372) (end 159.13 99.65) (width 0.2) (layer "B.Cu") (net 24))
 (segment (start 186.79 27) (end 186.79 56.0402) (width 0.2) (layer "B.Cu") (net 24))
 (segment (start 175.5429 67.2873) (end 175.5429 83.2372) (width 0.2) (layer "B.Cu") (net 24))
 (segment (start 175.5429 83.2372) (end 175.5428 83.2372) (width 0.2) (layer "B.Cu") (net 24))
 (segment (start 186.79 56.0402) (end 175.5429 67.2873) (width 0.2) (layer "B.Cu") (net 24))
 (segment (start 157.4894 103.0894) (end 159.13 104.73) (width 0.2) (layer "B.Cu") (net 26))
 (segment (start 181.71 27) (end 181.71 59.4259) (width 0.2) (layer "B.Cu") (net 26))
 (segment (start 157.4894 83.6465) (end 157.4894 103.0894) (width 0.2) (layer "B.Cu") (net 26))
 (segment (start 181.71 59.4259) (end 157.4894 83.6465) (width 0.2) (layer "B.Cu") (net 26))
 (segment (start 165.15 63.9916) (end 163.88 62.7216) (width 0.2) (layer "F.Cu") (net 15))
 (segment (start 163.88 62.7216) (end 163.88 54.5) (width 0.2) (layer "F.Cu") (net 15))
 (segment (start 166.6051 99.5051) (end 166.6051 67.3399) (width 0.2) (layer "F.Cu") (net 15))
 (segment (start 165.15 65.8848) (end 165.15 63.9916) (width 0.2) (layer "F.Cu") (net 15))
 (segment (start 166.6051 67.3399) (end 165.15 65.8848) (width 0.2) (layer "F.Cu") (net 15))
 (segment (start 174.37 107.27) (end 166.6051 99.5051) (width 0.2) (layer "F.Cu") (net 15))
 (segment (start 174.37 97.11) (end 178.75 92.73) (width 0.2) (layer "B.Cu") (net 12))
 (segment (start 178.75 92.73) (end 178.75 87.5) (width 0.2) (layer "B.Cu") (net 12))
 (segment (start 191.25 87.5) (end 189.3483 87.5) (width 0.2) (layer "B.Cu") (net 12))
 (segment (start 178.75 87.5) (end 189.3483 87.5) (width 0.2) (layer "B.Cu") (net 12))
 (segment (start 162.5717 28.9017) (end 162.5717 28) (width 0.2) (layer "F.Cu") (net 11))
 (segment (start 173.8613 105.908) (end 167.69 99.7367) (width 0.2) (layer "F.Cu") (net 11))
 (segment (start 175.5576 106.7107) (end 174.7549 105.908) (width 0.2) (layer "F.Cu") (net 11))
 (segment (start 174.37 117.43) (end 175.5576 116.2424) (width 0.2) (layer "F.Cu") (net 11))
 (segment (start 167.69 99.7367) (end 167.69 34.02) (width 0.2) (layer "F.Cu") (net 11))
 (segment (start 161.67 28) (end 162.5717 28) (width 0.2) (layer "F.Cu") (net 11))
 (segment (start 174.7549 105.908) (end 173.8613 105.908) (width 0.2) (layer "F.Cu") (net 11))
 (segment (start 167.69 34.02) (end 162.5717 28.9017) (width 0.2) (layer "F.Cu") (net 11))
 (segment (start 175.5576 116.2424) (end 175.5576 106.7107) (width 0.2) (layer "F.Cu") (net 11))
 (segment (start 161.34 62.2027) (end 161.34 54.5) (width 0.2) (layer "F.Cu") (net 14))
 (segment (start 166.2034 69.1564) (end 162.8163 65.7693) (width 0.2) (layer "F.Cu") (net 14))
 (segment (start 162.8163 65.7693) (end 162.8163 63.679) (width 0.2) (layer "F.Cu") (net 14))
 (segment (start 162.8163 63.679) (end 161.34 62.2027) (width 0.2) (layer "F.Cu") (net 14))
 (segment (start 166.2034 101.6434) (end 166.2034 69.1564) (width 0.2) (layer "F.Cu") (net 14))
 (segment (start 174.37 109.81) (end 166.2034 101.6434) (width 0.2) (layer "F.Cu") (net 14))
 (segment (start 175.9704 117.5597) (end 174.7381 118.792) (width 0.2) (layer "F.Cu") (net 9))
 (segment (start 175.9704 102.1229) (end 175.9704 117.5597) (width 0.2) (layer "F.Cu") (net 9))
 (segment (start 173.8821 100.92) (end 174.7675 100.92) (width 0.2) (layer "F.Cu") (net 9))
 (segment (start 174.37 119.97) (end 174.37 118.792) (width 0.2) (layer "F.Cu") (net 9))
 (segment (start 174.7675 100.92) (end 175.9704 102.1229) (width 0.2) (layer "F.Cu") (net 9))
 (segment (start 166.75 28) (end 167.6517 28) (width 0.2) (layer "F.Cu") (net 9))
 (segment (start 174.7381 118.792) (end 174.37 118.792) (width 0.2) (layer "F.Cu") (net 9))
 (segment (start 167.6517 28) (end 170.4116 30.7599) (width 0.2) (layer "F.Cu") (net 9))
 (segment (start 170.4116 30.7599) (end 170.4116 97.4495) (width 0.2) (layer "F.Cu") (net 9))
 (segment (start 170.4116 97.4495) (end 173.8821 100.92) (width 0.2) (layer "F.Cu") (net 9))
 (segment (start 174.37 94.57) (end 176.8483 92.0917) (width 0.2) (layer "B.Cu") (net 19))
 (segment (start 191.25 67.25) (end 178.75 67.25) (width 0.2) (layer "B.Cu") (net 19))
 (segment (start 176.8483 92.0917) (end 176.8483 67.25) (width 0.2) (layer "B.Cu") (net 19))
 (segment (start 178.75 67.25) (end 176.8483 67.25) (width 0.2) (layer "B.Cu") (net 19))
 (segment (start 176.8483 97.75) (end 176.8483 99.7117) (width 0.2) (layer "B.Cu") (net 17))
 (segment (start 176.8483 99.7117) (end 174.37 102.19) (width 0.2) (layer "B.Cu") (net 17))
 (segment (start 178.75 97.75) (end 176.8483 97.75) (width 0.2) (layer "B.Cu") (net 17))
 (segment (start 191.25 97.75) (end 178.75 97.75) (width 0.2) (layer "B.Cu") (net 17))
 (segment (start 167.128 26.6733) (end 166.3417 26.6733) (width 0.2) (layer "F.Cu") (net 10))
 (segment (start 178.75 72.25) (end 180.6517 72.25) (width 0.2) (layer "F.Cu") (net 10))
 (segment (start 178.75 51.75) (end 179.7009 51.75) (width 0.2) (layer "F.Cu") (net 10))
 (segment (start 191.25 72.25) (end 189.3483 72.25) (width 0.2) (layer "F.Cu") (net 10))
 (segment (start 165.1117 27.9033) (end 165.1117 28) (width 0.2) (layer "F.Cu") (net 10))
 (segment (start 191.25 113.25) (end 193.1517 113.25) (width 0.2) (layer "F.Cu") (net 10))
 (segment (start 178.75 102.75) (end 180.5509 102.75) (width 0.2) (layer "F.Cu") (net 10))
 (segment (start 180.6517 102.7485) (end 180.6517 82.5) (width 0.2) (layer "F.Cu") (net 10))
 (segment (start 191.25 102.75) (end 192.2009 102.75) (width 0.2) (layer "F.Cu") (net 10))
 (segment (start 180.6502 102.75) (end 180.6517 102.75) (width 0.2) (layer "F.Cu") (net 10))
 (segment (start 179.7009 51.75) (end 180.6517 51.75) (width 0.2) (layer "F.Cu") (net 10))
 (segment (start 180.6517 102.75) (end 180.6517 113.25) (width 0.2) (layer "F.Cu") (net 10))
 (segment (start 179.2255 40.75) (end 179.7009 40.75) (width 0.2) (layer "F.Cu") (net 10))
 (segment (start 189.3483 82.5) (end 180.6517 82.5) (width 0.2) (layer "F.Cu") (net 10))
 (segment (start 191.25 51.75) (end 193.1517 51.75) (width 0.2) (layer "F.Cu") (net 10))
 (segment (start 193.1517 112.7315) (end 193.1517 113.25) (width 0.2) (layer "F.Cu") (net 10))
 (segment (start 191.25 82.5) (end 189.3483 82.5) (width 0.2) (layer "F.Cu") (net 10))
 (segment (start 191.25 72.25) (end 193.1517 72.25) (width 0.2) (layer "F.Cu") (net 10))
 (segment (start 179.7009 40.75) (end 180.6517 40.75) (width 0.2) (layer "F.Cu") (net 10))
 (segment (start 180.6502 102.75) (end 180.6517 102.7485) (width 0.2) (layer "F.Cu") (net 10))
 (segment (start 180.5509 102.75) (end 180.6502 102.75) (width 0.2) (layer "F.Cu") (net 10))
 (segment (start 192.2009 111.7808) (end 192.201 111.7808) (width 0.2) (layer "F.Cu") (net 10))
 (segment (start 192.2009 102.75) (end 192.2009 111.7808) (width 0.2) (layer "F.Cu") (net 10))
 (segment (start 164.21 28) (end 165.1117 28) (width 0.2) (layer "F.Cu") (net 10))
 (segment (start 178.75 113.25) (end 180.6517 113.25) (width 0.2) (layer "F.Cu") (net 10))
 (segment (start 191.25 113.25) (end 180.6517 113.25) (width 0.2) (layer "F.Cu") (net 10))
 (segment (start 180.6517 51.75) (end 191.25 51.75) (width 0.2) (layer "F.Cu") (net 10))
 (segment (start 178.75 40.75) (end 179.2255 40.75) (width 0.2) (layer "F.Cu") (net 10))
 (segment (start 180.6517 72.25) (end 180.6517 82.5) (width 0.2) (layer "F.Cu") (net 10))
 (segment (start 179.2255 38.7708) (end 167.128 26.6733) (width 0.2) (layer "F.Cu") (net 10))
 (segment (start 166.3417 26.6733) (end 165.1117 27.9033) (width 0.2) (layer "F.Cu") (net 10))
 (segment (start 179.2255 40.75) (end 179.2255 38.7708) (width 0.2) (layer "F.Cu") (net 10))
 (segment (start 192.201 111.7808) (end 193.1517 112.7315) (width 0.2) (layer "F.Cu") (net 10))
 (segment (start 180.6517 40.75) (end 191.25 40.75) (width 0.2) (layer "F.Cu") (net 10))
 (segment (start 193.1517 51.75) (end 193.1517 72.25) (width 0.2) (layer "F.Cu") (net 10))
 (segment (start 178.75 82.5) (end 180.6517 82.5) (width 0.2) (layer "F.Cu") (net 10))
 (segment (start 180.6517 40.75) (end 180.6517 51.75) (width 0.2) (layer "F.Cu") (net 10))
 (segment (start 189.3483 82.5) (end 189.3483 72.25) (width 0.2) (layer "F.Cu") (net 10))
 (segment (start 178.75 113.25) (end 176.8483 113.25) (width 0.2) (layer "B.Cu") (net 10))
 (segment (start 175.2083 114.89) (end 176.8483 113.25) (width 0.2) (layer "B.Cu") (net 10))
 (segment (start 174.37 114.89) (end 175.2083 114.89) (width 0.2) (layer "B.Cu") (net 10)))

